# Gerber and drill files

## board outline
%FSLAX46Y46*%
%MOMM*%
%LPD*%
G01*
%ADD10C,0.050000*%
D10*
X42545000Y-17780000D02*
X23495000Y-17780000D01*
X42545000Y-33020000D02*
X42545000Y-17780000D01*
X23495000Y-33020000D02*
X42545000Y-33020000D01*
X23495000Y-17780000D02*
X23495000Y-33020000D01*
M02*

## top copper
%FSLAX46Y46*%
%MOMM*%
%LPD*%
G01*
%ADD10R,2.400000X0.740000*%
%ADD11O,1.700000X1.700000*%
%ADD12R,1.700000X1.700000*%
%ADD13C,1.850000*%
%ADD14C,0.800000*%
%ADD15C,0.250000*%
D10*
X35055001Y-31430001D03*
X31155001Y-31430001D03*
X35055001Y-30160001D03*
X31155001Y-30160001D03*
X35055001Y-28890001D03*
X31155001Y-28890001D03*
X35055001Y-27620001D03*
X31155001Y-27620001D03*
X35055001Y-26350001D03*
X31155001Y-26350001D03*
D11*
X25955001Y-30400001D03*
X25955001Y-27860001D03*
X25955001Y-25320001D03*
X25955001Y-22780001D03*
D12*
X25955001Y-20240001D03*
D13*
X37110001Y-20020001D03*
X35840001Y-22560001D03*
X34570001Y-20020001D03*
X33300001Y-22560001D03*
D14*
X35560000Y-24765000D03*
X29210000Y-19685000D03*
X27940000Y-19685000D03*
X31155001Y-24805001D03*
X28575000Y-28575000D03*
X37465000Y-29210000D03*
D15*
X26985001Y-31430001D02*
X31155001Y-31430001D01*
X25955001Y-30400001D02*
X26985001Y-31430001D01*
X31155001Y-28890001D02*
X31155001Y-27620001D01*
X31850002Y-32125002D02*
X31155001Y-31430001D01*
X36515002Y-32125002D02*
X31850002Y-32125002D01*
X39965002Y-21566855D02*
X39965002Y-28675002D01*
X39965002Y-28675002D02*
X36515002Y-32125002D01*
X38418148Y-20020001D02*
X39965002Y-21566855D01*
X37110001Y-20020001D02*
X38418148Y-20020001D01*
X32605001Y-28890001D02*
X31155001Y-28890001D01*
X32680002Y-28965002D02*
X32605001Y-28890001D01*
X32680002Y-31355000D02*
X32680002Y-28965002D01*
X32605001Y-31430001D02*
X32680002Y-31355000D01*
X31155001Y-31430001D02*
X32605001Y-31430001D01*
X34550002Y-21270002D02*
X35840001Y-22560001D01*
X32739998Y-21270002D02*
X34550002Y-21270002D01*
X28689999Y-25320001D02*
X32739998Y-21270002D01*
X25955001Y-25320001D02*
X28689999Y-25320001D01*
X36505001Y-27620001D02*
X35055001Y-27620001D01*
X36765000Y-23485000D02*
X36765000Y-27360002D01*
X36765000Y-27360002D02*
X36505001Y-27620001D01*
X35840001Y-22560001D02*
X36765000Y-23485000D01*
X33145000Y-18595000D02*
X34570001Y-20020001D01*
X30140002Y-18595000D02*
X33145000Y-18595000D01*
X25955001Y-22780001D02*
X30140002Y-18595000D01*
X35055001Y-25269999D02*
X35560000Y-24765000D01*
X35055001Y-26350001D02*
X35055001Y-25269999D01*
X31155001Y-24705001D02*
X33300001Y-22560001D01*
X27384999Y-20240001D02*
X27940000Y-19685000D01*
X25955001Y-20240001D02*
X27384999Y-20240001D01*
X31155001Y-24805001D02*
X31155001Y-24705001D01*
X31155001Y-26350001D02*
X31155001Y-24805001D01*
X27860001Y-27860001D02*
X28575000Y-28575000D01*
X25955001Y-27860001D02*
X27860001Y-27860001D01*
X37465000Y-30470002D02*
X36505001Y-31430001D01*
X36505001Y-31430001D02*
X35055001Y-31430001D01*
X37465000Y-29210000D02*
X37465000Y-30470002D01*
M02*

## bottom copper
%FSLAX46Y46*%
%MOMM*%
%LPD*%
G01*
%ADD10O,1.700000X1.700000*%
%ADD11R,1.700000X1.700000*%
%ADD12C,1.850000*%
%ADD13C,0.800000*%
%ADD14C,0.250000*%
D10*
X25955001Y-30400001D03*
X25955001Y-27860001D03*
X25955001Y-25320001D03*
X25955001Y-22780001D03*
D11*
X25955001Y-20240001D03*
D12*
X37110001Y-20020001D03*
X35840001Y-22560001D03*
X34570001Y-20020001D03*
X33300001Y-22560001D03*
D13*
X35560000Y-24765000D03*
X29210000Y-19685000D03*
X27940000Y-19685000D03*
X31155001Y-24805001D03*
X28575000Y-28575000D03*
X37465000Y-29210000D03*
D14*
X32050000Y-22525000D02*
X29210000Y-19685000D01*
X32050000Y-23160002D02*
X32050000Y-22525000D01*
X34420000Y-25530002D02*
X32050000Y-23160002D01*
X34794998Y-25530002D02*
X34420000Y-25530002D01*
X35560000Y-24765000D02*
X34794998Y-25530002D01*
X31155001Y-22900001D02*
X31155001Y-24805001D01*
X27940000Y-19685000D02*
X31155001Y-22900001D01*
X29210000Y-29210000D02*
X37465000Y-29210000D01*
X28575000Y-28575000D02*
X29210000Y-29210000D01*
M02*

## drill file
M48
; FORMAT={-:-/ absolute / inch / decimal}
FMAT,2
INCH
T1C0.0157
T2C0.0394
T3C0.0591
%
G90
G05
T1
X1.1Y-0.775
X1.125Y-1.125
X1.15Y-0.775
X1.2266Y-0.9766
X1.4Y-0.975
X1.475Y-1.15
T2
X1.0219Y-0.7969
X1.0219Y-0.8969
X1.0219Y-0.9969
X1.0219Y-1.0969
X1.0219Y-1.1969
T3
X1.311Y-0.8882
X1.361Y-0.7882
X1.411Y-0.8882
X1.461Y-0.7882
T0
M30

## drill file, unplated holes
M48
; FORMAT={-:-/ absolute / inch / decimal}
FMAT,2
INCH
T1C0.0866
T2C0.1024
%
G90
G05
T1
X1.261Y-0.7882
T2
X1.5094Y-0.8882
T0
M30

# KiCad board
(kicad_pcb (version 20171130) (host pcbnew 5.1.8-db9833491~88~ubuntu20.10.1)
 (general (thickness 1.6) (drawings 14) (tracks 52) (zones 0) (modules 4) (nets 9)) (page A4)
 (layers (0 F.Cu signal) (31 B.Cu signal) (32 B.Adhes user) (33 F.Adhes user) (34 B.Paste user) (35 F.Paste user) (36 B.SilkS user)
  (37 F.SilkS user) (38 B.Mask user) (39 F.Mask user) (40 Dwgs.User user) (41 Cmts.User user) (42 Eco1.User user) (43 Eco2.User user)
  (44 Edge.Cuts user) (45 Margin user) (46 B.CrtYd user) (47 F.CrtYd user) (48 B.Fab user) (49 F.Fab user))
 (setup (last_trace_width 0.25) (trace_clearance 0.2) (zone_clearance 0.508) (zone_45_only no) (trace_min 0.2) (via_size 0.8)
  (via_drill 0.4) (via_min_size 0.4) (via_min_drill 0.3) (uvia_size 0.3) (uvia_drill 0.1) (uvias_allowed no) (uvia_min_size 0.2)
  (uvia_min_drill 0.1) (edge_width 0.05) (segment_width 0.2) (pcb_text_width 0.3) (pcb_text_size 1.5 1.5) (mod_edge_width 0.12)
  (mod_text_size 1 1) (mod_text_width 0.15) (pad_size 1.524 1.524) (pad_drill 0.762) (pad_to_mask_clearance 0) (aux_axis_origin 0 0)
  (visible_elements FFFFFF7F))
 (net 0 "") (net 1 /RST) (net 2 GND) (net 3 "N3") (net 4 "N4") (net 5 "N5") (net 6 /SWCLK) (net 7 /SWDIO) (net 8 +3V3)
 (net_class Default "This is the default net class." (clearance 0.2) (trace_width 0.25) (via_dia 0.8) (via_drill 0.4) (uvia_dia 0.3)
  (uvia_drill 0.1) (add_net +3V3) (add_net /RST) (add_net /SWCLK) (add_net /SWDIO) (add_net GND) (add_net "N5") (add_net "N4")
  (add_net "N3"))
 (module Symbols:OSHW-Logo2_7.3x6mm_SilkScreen (layer B.Cu) (at 33.655 29.21 180)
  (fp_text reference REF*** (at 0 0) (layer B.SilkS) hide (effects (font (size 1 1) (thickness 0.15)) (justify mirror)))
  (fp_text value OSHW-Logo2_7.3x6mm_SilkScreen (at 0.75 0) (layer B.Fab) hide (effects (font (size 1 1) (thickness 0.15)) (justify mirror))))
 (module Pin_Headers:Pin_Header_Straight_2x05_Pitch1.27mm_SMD (layer F.Cu) (at 33.105001 28.890001)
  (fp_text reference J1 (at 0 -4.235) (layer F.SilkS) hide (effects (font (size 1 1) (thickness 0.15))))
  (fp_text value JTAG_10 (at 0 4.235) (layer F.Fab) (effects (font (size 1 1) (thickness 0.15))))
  (pad 10 smd rect (at 1.95 2.54) (size 2.4 0.74) (layers F.Cu F.Paste F.Mask) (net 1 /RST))
  (pad 9 smd rect (at -1.95 2.54) (size 2.4 0.74) (layers F.Cu F.Paste F.Mask) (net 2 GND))
  (pad 8 smd rect (at 1.95 1.27) (size 2.4 0.74) (layers F.Cu F.Paste F.Mask) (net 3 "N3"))
  (pad 7 smd rect (at -1.95 1.27) (size 2.4 0.74) (layers F.Cu F.Paste F.Mask) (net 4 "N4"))
  (pad 6 smd rect (at 1.95 0) (size 2.4 0.74) (layers F.Cu F.Paste F.Mask) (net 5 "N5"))
  (pad 5 smd rect (at -1.95 0) (size 2.4 0.74) (layers F.Cu F.Paste F.Mask) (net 2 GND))
  (pad 4 smd rect (at 1.95 -1.27) (size 2.4 0.74) (layers F.Cu F.Paste F.Mask) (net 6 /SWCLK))
  (pad 3 smd rect (at -1.95 -1.27) (size 2.4 0.74) (layers F.Cu F.Paste F.Mask) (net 2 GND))
  (pad 2 smd rect (at 1.95 -2.54) (size 2.4 0.74) (layers F.Cu F.Paste F.Mask) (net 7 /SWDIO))
  (pad 1 smd rect (at -1.95 -2.54) (size 2.4 0.74) (layers F.Cu F.Paste F.Mask) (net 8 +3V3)))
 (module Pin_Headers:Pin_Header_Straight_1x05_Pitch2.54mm (layer F.Cu) (at 25.955001 20.240001)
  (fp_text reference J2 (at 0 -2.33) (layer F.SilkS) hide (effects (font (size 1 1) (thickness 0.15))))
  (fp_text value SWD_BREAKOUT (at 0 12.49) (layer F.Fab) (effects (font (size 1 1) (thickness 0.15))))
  (pad 5 thru_hole oval (at 0 10.16) (size 1.7 1.7) (drill 1) (layers *.Cu *.Mask) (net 2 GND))
  (pad 4 thru_hole oval (at 0 7.62) (size 1.7 1.7) (drill 1) (layers *.Cu *.Mask) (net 1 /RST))
  (pad 3 thru_hole oval (at 0 5.08) (size 1.7 1.7) (drill 1) (layers *.Cu *.Mask) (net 6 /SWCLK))
  (pad 2 thru_hole oval (at 0 2.54) (size 1.7 1.7) (drill 1) (layers *.Cu *.Mask) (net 7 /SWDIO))
  (pad 1 thru_hole rect (at 0 0) (size 1.7 1.7) (drill 1) (layers *.Cu *.Mask) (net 8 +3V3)))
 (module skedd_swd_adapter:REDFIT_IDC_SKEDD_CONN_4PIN (layer F.Cu) (at 35.205001 21.290001)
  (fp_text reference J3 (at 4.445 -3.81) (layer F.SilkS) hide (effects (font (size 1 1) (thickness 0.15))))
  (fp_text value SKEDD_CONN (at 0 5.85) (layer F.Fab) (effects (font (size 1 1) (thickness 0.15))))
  (pad "" np_thru_hole circle (at 3.135 1.27) (size 2.6 2.6) (drill 2.6) (layers *.Cu *.Mask))
  (pad "" np_thru_hole circle (at -3.175 -1.27) (size 2.2 2.2) (drill 2.2) (layers *.Cu *.Mask))
  (pad 4 thru_hole circle (at 1.905 -1.27) (size 1.85 1.85) (drill 1.5) (layers *.Cu *.Mask) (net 2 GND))
  (pad 3 thru_hole circle (at 0.635 1.27) (size 1.85 1.85) (drill 1.5) (layers *.Cu *.Mask) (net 6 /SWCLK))
  (pad 2 thru_hole circle (at -0.635 -1.27) (size 1.85 1.85) (drill 1.5) (layers *.Cu *.Mask) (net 7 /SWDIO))
  (pad 1 thru_hole circle (at -1.905 1.27) (size 1.85 1.85) (drill 1.5) (layers *.Cu *.Mask) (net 8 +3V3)))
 (gr_line (start 42.545 17.78) (end 23.495 17.78) (layer Edge.Cuts) (width 0.05))
 (gr_line (start 42.545 33.02) (end 42.545 17.78) (layer Edge.Cuts) (width 0.05))
 (gr_line (start 23.495 33.02) (end 42.545 33.02) (layer Edge.Cuts) (width 0.05))
 (gr_line (start 23.495 17.78) (end 23.495 33.02) (layer Edge.Cuts) (width 0.05))
 (segment (start 26.985001 31.430001) (end 31.155001 31.430001) (width 0.25) (layer F.Cu) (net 2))
 (segment (start 25.955001 30.400001) (end 26.985001 31.430001) (width 0.25) (layer F.Cu) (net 2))
 (segment (start 31.155001 28.890001) (end 31.155001 27.620001) (width 0.25) (layer F.Cu) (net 2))
 (segment (start 31.850002 32.125002) (end 31.155001 31.430001) (width 0.25) (layer F.Cu) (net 2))
 (segment (start 36.515002 32.125002) (end 31.850002 32.125002) (width 0.25) (layer F.Cu) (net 2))
 (segment (start 39.965002 21.566855) (end 39.965002 28.675002) (width 0.25) (layer F.Cu) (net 2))
 (segment (start 39.965002 28.675002) (end 36.515002 32.125002) (width 0.25) (layer F.Cu) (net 2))
 (segment (start 38.418148 20.020001) (end 39.965002 21.566855) (width 0.25) (layer F.Cu) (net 2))
 (segment (start 37.110001 20.020001) (end 38.418148 20.020001) (width 0.25) (layer F.Cu) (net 2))
 (segment (start 32.605001 28.890001) (end 31.155001 28.890001) (width 0.25) (layer F.Cu) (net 2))
 (segment (start 32.680002 28.965002) (end 32.605001 28.890001) (width 0.25) (layer F.Cu) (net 2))
 (segment (start 32.680002 31.355) (end 32.680002 28.965002) (width 0.25) (layer F.Cu) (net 2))
 (segment (start 32.605001 31.430001) (end 32.680002 31.355) (width 0.25) (layer F.Cu) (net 2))
 (segment (start 31.155001 31.430001) (end 32.605001 31.430001) (width 0.25) (layer F.Cu) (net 2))
 (segment (start 34.550002 21.270002) (end 35.840001 22.560001) (width 0.25) (layer F.Cu) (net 6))
 (segment (start 32.739998 21.270002) (end 34.550002 21.270002) (width 0.25) (layer F.Cu) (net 6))
 (segment (start 28.689999 25.320001) (end 32.739998 21.270002) (width 0.25) (layer F.Cu) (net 6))
 (segment (start 25.955001 25.320001) (end 28.689999 25.320001) (width 0.25) (layer F.Cu) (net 6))
 (segment (start 36.505001 27.620001) (end 35.055001 27.620001) (width 0.25) (layer F.Cu) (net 6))
 (segment (start 36.765 23.485) (end 36.765 27.360002) (width 0.25) (layer F.Cu) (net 6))
 (segment (start 36.765 27.360002) (end 36.505001 27.620001) (width 0.25) (layer F.Cu) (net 6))
 (segment (start 35.840001 22.560001) (end 36.765 23.485) (width 0.25) (layer F.Cu) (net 6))
 (segment (start 33.145 18.595) (end 34.570001 20.020001) (width 0.25) (layer F.Cu) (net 7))
 (segment (start 30.140002 18.595) (end 33.145 18.595) (width 0.25) (layer F.Cu) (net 7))
 (segment (start 25.955001 22.780001) (end 30.140002 18.595) (width 0.25) (layer F.Cu) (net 7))
 (via (at 35.56 24.765) (size 0.8) (drill 0.4) (layers F.Cu B.Cu) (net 7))
 (segment (start 35.055001 25.269999) (end 35.56 24.765) (width 0.25) (layer F.Cu) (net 7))
 (segment (start 35.055001 26.350001) (end 35.055001 25.269999) (width 0.25) (layer F.Cu) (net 7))
 (via (at 29.21 19.685) (size 0.8) (drill 0.4) (layers F.Cu B.Cu) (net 7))
 (segment (start 32.05 22.525) (end 29.21 19.685) (width 0.25) (layer B.Cu) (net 7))
 (segment (start 32.05 23.160002) (end 32.05 22.525) (width 0.25) (layer B.Cu) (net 7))
 (segment (start 34.42 25.530002) (end 32.05 23.160002) (width 0.25) (layer B.Cu) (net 7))
 (segment (start 34.794998 25.530002) (end 34.42 25.530002) (width 0.25) (layer B.Cu) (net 7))
 (segment (start 35.56 24.765) (end 34.794998 25.530002) (width 0.25) (layer B.Cu) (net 7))
 (segment (start 31.155001 24.705001) (end 33.300001 22.560001) (width 0.25) (layer F.Cu) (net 8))
 (via (at 27.94 19.685) (size 0.8) (drill 0.4) (layers F.Cu B.Cu) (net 8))
 (segment (start 27.384999 20.240001) (end 27.94 19.685) (width 0.25) (layer F.Cu) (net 8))
 (segment (start 25.955001 20.240001) (end 27.384999 20.240001) (width 0.25) (layer F.Cu) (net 8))
 (via (at 31.155001 24.805001) (size 0.8) (drill 0.4) (layers F.Cu B.Cu) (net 8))
 (segment (start 31.155001 22.900001) (end 31.155001 24.805001) (width 0.25) (layer B.Cu) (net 8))
 (segment (start 27.94 19.685) (end 31.155001 22.900001) (width 0.25) (layer B.Cu) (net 8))
 (segment (start 31.155001 24.805001) (end 31.155001 24.705001) (width 0.25) (layer F.Cu) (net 8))
 (segment (start 31.155001 26.350001) (end 31.155001 24.805001) (width 0.25) (layer F.Cu) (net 8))
 (via (at 28.575 28.575) (size 0.8) (drill 0.4) (layers F.Cu B.Cu) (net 1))
 (segment (start 27.860001 27.860001) (end 28.575 28.575) (width 0.25) (layer F.Cu) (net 1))
 (segment (start 25.955001 27.860001) (end 27.860001 27.860001) (width 0.25) (layer F.Cu) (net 1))
 (via (at 37.465 29.21) (size 0.8) (drill 0.4) (layers F.Cu B.Cu) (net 1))
 (segment (start 29.21 29.21) (end 37.465 29.21) (width 0.25) (layer B.Cu) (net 1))
 (segment (start 28.575 28.575) (end 29.21 29.21) (width 0.25) (layer B.Cu) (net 1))
 (segment (start 37.465 30.470002) (end 36.505001 31.430001) (width 0.25) (layer F.Cu) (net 1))
 (segment (start 36.505001 31.430001) (end 35.055001 31.430001) (width 0.25) (layer F.Cu) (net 1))
 (segment (start 37.465 29.21) (end 37.465 30.470002) (width 0.25) (layer F.Cu) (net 1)))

